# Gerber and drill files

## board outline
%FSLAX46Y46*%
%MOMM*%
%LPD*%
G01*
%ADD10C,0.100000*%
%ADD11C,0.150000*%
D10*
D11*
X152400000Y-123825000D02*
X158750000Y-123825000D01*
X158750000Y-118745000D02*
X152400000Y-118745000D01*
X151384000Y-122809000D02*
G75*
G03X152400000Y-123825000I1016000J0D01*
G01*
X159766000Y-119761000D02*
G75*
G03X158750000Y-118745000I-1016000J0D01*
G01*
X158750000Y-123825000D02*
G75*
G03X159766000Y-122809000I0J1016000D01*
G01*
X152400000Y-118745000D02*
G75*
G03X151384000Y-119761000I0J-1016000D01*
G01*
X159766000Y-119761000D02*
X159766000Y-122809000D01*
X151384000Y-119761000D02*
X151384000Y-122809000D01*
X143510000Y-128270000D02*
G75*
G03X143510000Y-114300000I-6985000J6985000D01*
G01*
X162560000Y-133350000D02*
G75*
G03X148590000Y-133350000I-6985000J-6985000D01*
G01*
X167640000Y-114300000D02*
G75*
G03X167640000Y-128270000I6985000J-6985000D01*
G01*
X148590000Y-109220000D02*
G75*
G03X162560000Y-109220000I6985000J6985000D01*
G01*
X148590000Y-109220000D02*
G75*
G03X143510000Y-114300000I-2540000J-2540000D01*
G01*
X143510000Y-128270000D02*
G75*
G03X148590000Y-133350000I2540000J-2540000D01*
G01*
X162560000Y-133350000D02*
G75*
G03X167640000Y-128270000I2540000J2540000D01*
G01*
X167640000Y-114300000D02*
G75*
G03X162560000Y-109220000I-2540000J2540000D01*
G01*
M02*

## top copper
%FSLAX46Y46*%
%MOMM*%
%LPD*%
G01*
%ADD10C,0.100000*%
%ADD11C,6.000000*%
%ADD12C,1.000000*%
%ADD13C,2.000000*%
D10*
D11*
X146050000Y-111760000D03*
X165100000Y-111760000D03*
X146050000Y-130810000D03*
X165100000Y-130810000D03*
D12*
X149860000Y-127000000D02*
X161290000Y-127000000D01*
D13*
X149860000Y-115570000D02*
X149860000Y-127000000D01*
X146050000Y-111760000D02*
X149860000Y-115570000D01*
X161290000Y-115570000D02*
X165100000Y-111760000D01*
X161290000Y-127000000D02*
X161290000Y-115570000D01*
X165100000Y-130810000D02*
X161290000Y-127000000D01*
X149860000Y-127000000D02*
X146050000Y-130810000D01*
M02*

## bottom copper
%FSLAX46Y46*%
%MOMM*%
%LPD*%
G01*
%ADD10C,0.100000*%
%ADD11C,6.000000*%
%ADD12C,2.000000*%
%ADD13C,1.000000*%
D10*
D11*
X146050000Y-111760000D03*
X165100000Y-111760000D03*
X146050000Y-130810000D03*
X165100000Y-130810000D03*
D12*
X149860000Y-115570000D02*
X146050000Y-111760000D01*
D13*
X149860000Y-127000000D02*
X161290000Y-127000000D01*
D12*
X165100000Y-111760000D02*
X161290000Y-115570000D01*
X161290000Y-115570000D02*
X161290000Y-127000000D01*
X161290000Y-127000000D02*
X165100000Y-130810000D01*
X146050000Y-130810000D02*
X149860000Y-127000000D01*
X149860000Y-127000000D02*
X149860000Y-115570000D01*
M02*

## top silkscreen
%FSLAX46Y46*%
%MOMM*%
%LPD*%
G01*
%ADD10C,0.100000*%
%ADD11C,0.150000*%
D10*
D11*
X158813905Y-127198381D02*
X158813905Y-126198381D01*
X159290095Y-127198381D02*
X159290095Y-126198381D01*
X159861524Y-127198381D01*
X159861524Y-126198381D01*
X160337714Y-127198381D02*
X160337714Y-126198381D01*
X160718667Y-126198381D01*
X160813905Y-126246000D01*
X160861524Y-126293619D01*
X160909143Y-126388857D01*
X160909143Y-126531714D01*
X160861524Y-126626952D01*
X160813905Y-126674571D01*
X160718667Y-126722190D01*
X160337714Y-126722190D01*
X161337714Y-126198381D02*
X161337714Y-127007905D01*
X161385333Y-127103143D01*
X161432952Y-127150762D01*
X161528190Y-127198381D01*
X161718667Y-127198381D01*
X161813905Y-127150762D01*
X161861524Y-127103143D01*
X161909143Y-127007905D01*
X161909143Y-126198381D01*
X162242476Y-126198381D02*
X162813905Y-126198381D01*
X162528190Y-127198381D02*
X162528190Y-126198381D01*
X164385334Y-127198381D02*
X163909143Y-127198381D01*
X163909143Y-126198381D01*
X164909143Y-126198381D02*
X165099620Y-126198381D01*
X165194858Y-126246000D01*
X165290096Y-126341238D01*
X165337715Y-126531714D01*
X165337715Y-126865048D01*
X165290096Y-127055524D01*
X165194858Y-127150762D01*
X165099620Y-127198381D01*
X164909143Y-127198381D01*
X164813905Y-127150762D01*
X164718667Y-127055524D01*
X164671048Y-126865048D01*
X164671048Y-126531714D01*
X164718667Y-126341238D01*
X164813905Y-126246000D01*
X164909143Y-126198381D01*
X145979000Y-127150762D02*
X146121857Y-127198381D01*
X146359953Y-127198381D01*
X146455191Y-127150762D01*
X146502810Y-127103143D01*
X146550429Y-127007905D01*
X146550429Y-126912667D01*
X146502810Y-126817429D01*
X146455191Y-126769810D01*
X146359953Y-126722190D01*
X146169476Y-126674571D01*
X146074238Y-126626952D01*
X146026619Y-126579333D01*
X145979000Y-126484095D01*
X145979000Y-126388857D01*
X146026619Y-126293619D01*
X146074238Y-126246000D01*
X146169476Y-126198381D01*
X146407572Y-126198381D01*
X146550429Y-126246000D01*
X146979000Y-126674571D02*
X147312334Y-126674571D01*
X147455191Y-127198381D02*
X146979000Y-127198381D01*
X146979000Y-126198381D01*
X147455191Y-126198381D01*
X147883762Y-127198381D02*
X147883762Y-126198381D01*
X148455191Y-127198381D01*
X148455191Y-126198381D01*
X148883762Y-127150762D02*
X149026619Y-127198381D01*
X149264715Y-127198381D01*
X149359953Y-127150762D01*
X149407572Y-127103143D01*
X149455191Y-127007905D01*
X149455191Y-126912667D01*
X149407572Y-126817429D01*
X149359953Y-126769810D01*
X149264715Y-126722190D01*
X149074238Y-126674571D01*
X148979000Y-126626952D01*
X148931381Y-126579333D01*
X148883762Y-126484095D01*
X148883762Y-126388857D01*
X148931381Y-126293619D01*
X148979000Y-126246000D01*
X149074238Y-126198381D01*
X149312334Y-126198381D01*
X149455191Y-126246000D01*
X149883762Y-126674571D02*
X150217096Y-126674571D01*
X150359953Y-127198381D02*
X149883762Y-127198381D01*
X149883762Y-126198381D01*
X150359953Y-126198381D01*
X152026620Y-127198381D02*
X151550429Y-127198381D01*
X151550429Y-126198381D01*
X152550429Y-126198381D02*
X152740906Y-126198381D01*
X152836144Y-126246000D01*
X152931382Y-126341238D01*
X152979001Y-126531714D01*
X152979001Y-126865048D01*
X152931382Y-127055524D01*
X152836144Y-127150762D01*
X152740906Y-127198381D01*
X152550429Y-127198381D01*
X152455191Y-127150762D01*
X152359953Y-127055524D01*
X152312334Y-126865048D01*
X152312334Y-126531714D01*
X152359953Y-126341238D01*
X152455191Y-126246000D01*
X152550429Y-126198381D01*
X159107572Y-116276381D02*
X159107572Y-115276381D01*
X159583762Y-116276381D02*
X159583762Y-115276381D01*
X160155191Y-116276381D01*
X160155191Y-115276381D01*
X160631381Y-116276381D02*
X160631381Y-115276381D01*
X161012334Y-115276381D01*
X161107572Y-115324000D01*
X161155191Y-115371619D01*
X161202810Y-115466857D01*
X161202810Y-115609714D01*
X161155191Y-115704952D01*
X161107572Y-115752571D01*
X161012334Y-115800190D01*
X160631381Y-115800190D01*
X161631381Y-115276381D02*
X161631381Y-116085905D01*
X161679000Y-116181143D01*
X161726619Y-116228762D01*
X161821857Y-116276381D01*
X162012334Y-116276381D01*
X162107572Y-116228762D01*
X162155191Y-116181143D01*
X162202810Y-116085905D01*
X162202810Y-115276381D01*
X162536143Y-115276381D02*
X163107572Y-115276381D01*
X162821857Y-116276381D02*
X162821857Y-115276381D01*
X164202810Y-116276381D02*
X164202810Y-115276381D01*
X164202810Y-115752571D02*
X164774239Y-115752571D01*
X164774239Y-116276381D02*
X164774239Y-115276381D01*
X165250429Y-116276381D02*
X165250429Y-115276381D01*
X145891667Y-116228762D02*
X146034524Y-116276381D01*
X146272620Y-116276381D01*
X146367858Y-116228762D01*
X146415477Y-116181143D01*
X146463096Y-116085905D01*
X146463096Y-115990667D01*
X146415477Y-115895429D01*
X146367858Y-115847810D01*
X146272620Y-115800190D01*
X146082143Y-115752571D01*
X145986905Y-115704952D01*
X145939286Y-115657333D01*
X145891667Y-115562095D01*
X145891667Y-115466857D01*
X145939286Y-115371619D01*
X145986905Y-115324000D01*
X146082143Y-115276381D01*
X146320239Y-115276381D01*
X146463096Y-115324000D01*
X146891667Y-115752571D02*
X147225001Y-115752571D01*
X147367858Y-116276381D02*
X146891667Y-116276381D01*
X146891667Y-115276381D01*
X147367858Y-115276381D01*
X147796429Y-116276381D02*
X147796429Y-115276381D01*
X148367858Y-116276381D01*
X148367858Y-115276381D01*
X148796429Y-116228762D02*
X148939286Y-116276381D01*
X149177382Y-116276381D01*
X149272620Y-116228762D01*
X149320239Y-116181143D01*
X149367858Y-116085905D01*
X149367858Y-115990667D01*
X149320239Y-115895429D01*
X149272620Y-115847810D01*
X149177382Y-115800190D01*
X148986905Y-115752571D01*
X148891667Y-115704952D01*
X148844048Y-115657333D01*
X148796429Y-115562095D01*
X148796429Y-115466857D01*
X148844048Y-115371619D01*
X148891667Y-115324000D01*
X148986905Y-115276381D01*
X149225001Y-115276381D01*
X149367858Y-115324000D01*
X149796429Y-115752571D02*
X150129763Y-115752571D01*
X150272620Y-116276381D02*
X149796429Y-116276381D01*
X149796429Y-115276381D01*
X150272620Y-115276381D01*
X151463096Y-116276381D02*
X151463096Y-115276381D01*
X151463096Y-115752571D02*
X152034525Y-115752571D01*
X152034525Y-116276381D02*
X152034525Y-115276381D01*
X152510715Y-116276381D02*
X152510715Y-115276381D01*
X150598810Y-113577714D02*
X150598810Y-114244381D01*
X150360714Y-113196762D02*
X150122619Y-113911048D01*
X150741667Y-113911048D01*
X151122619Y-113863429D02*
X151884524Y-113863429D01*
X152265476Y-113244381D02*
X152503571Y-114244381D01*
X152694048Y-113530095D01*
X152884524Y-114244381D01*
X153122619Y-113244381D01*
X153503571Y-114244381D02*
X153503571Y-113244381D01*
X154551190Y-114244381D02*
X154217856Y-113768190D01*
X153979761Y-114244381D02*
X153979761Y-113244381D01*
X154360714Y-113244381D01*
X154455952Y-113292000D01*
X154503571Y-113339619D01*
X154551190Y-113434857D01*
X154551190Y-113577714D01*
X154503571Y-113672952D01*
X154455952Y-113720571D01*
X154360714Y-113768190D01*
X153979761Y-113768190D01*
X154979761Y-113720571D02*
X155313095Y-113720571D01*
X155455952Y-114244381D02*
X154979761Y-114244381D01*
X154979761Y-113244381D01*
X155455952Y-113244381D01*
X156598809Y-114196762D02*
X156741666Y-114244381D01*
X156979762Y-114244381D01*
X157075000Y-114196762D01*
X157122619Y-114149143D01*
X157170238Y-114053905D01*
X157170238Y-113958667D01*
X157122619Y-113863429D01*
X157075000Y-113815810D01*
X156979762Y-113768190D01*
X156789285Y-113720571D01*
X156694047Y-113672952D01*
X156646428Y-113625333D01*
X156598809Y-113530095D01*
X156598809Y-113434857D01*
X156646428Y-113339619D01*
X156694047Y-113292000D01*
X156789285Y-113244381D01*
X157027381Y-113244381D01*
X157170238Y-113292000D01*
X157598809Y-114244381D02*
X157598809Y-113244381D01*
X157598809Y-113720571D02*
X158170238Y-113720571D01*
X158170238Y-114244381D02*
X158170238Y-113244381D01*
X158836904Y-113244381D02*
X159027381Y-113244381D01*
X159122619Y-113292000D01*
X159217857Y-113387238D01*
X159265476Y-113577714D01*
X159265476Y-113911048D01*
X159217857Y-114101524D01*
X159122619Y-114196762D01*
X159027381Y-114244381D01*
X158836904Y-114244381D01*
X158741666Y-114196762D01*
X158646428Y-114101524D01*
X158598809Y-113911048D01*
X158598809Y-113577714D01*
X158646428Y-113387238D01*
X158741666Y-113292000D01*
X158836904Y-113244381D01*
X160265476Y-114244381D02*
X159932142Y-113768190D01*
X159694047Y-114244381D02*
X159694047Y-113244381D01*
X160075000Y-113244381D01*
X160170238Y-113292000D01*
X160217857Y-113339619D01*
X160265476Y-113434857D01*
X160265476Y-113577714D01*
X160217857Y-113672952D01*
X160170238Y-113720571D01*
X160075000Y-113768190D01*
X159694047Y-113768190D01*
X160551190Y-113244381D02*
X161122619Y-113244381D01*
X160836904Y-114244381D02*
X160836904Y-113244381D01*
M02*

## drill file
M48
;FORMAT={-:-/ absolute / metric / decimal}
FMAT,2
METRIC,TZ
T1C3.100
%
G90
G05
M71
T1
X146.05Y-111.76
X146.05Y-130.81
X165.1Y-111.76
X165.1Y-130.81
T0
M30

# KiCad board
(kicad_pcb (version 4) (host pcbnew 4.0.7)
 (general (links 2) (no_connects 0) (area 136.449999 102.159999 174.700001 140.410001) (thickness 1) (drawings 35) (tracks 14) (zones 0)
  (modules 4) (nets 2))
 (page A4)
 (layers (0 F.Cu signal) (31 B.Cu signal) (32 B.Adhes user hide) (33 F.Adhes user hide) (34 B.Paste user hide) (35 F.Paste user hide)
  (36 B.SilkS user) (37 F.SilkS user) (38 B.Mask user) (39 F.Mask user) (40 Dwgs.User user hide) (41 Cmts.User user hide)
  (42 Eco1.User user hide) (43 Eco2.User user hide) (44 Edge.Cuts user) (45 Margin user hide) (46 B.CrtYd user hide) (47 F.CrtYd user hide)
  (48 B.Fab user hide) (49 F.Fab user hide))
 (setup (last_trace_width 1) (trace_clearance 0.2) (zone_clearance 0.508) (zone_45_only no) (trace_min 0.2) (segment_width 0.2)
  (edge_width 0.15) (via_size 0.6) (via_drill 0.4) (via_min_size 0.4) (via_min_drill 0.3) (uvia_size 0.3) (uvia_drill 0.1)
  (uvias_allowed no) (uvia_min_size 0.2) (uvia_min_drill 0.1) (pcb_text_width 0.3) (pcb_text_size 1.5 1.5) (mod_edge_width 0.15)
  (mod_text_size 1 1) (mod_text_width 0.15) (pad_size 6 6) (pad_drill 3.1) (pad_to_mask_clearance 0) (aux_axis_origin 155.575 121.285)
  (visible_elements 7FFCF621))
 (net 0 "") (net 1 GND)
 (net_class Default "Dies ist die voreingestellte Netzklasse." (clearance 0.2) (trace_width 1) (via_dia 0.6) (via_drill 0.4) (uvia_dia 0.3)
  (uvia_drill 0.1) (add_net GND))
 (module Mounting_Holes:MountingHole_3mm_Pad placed (layer F.Cu) (at 146.05 111.76)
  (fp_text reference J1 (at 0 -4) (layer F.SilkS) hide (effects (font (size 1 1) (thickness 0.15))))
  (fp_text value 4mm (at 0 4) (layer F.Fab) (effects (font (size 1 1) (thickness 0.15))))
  (pad 1 thru_hole circle (at 0 0) (size 6 6) (drill 3.1) (layers *.Cu *.Mask) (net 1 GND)))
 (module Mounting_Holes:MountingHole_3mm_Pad (layer F.Cu) (at 165.1 111.76)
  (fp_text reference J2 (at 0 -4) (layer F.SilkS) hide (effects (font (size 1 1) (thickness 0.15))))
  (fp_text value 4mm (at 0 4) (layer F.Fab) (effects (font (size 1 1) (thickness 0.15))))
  (pad 1 thru_hole circle (at 0 0) (size 6 6) (drill 3.1) (layers *.Cu *.Mask) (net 1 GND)))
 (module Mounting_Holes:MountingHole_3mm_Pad (layer F.Cu) (at 146.05 130.81)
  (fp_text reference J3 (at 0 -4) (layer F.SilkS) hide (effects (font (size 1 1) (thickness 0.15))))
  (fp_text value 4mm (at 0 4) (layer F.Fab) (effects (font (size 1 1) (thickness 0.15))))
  (pad 1 thru_hole circle (at 0 0) (size 6 6) (drill 3.1) (layers *.Cu *.Mask) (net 1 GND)))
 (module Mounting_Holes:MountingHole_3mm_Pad (layer F.Cu) (at 165.1 130.81)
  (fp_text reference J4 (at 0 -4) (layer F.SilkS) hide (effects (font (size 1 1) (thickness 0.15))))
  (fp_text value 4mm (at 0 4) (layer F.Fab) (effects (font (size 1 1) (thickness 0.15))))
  (pad 1 thru_hole circle (at 0 0) (size 6 6) (drill 3.1) (layers *.Cu *.Mask) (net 1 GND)))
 (gr_line (start 152.4 123.825) (end 158.75 123.825) (angle 90) (layer Edge.Cuts) (width 0.15))
 (gr_line (start 158.75 118.745) (end 152.4 118.745) (angle 90) (layer Edge.Cuts) (width 0.15))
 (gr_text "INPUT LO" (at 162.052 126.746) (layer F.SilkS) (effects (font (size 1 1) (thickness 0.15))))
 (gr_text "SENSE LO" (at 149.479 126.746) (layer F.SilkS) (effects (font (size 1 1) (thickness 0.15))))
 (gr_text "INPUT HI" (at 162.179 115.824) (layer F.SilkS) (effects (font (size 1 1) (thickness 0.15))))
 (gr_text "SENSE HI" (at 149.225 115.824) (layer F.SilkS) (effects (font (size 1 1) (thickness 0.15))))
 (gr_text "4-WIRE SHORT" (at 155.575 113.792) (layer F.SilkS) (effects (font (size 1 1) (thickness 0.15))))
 (gr_arc (start 152.4 122.809) (end 152.4 123.825) (angle 90) (layer Edge.Cuts) (width 0.15))
 (gr_arc (start 158.75 119.761) (end 158.75 118.745) (angle 90) (layer Edge.Cuts) (width 0.15))
 (gr_arc (start 158.75 122.809) (end 159.766 122.809) (angle 90) (layer Edge.Cuts) (width 0.15))
 (gr_arc (start 152.4 119.761) (end 151.384 119.761) (angle 90) (layer Edge.Cuts) (width 0.15))
 (gr_line (start 159.766 119.761) (end 159.766 122.809) (angle 90) (layer Edge.Cuts) (width 0.15))
 (gr_line (start 151.384 119.761) (end 151.384 122.809) (angle 90) (layer Edge.Cuts) (width 0.15))
 (gr_arc (start 136.525 121.285) (end 143.51 114.3) (angle 90) (layer Edge.Cuts) (width 0.15))
 (gr_arc (start 155.575 140.335) (end 148.59 133.35) (angle 90) (layer Edge.Cuts) (width 0.15))
 (gr_arc (start 174.625 121.285) (end 167.64 128.27) (angle 90) (layer Edge.Cuts) (width 0.15))
 (gr_arc (start 155.575 102.235) (end 162.56 109.22) (angle 90) (layer Edge.Cuts) (width 0.15))
 (gr_arc (start 146.05 111.76) (end 143.51 114.3) (angle 180) (layer Edge.Cuts) (width 0.15))
 (gr_arc (start 146.05 130.81) (end 148.59 133.35) (angle 180) (layer Edge.Cuts) (width 0.15))
 (gr_arc (start 165.1 130.81) (end 167.64 128.27) (angle 180) (layer Edge.Cuts) (width 0.15))
 (gr_arc (start 165.1 111.76) (end 162.56 109.22) (angle 180) (layer Edge.Cuts) (width 0.15))
 (segment (start 149.86 127) (end 161.29 127) (width 1) (layer F.Cu) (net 1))
 (segment (start 149.86 115.57) (end 149.86 127) (width 2) (layer F.Cu) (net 1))
 (segment (start 146.05 111.76) (end 149.86 115.57) (width 2) (layer F.Cu) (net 1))
 (segment (start 161.29 115.57) (end 165.1 111.76) (width 2) (layer F.Cu) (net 1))
 (segment (start 161.29 127) (end 161.29 115.57) (width 2) (layer F.Cu) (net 1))
 (segment (start 165.1 130.81) (end 161.29 127) (width 2) (layer F.Cu) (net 1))
 (segment (start 149.86 127) (end 146.05 130.81) (width 2) (layer F.Cu) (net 1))
 (segment (start 149.86 115.57) (end 146.05 111.76) (width 2) (layer B.Cu) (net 1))
 (segment (start 149.86 127) (end 161.29 127) (width 1) (layer B.Cu) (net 1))
 (segment (start 165.1 111.76) (end 161.29 115.57) (width 2) (layer B.Cu) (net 1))
 (segment (start 161.29 115.57) (end 161.29 127) (width 2) (layer B.Cu) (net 1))
 (segment (start 161.29 127) (end 165.1 130.81) (width 2) (layer B.Cu) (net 1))
 (segment (start 146.05 130.81) (end 149.86 127) (width 2) (layer B.Cu) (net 1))
 (segment (start 149.86 127) (end 149.86 115.57) (width 2) (layer B.Cu) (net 1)))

